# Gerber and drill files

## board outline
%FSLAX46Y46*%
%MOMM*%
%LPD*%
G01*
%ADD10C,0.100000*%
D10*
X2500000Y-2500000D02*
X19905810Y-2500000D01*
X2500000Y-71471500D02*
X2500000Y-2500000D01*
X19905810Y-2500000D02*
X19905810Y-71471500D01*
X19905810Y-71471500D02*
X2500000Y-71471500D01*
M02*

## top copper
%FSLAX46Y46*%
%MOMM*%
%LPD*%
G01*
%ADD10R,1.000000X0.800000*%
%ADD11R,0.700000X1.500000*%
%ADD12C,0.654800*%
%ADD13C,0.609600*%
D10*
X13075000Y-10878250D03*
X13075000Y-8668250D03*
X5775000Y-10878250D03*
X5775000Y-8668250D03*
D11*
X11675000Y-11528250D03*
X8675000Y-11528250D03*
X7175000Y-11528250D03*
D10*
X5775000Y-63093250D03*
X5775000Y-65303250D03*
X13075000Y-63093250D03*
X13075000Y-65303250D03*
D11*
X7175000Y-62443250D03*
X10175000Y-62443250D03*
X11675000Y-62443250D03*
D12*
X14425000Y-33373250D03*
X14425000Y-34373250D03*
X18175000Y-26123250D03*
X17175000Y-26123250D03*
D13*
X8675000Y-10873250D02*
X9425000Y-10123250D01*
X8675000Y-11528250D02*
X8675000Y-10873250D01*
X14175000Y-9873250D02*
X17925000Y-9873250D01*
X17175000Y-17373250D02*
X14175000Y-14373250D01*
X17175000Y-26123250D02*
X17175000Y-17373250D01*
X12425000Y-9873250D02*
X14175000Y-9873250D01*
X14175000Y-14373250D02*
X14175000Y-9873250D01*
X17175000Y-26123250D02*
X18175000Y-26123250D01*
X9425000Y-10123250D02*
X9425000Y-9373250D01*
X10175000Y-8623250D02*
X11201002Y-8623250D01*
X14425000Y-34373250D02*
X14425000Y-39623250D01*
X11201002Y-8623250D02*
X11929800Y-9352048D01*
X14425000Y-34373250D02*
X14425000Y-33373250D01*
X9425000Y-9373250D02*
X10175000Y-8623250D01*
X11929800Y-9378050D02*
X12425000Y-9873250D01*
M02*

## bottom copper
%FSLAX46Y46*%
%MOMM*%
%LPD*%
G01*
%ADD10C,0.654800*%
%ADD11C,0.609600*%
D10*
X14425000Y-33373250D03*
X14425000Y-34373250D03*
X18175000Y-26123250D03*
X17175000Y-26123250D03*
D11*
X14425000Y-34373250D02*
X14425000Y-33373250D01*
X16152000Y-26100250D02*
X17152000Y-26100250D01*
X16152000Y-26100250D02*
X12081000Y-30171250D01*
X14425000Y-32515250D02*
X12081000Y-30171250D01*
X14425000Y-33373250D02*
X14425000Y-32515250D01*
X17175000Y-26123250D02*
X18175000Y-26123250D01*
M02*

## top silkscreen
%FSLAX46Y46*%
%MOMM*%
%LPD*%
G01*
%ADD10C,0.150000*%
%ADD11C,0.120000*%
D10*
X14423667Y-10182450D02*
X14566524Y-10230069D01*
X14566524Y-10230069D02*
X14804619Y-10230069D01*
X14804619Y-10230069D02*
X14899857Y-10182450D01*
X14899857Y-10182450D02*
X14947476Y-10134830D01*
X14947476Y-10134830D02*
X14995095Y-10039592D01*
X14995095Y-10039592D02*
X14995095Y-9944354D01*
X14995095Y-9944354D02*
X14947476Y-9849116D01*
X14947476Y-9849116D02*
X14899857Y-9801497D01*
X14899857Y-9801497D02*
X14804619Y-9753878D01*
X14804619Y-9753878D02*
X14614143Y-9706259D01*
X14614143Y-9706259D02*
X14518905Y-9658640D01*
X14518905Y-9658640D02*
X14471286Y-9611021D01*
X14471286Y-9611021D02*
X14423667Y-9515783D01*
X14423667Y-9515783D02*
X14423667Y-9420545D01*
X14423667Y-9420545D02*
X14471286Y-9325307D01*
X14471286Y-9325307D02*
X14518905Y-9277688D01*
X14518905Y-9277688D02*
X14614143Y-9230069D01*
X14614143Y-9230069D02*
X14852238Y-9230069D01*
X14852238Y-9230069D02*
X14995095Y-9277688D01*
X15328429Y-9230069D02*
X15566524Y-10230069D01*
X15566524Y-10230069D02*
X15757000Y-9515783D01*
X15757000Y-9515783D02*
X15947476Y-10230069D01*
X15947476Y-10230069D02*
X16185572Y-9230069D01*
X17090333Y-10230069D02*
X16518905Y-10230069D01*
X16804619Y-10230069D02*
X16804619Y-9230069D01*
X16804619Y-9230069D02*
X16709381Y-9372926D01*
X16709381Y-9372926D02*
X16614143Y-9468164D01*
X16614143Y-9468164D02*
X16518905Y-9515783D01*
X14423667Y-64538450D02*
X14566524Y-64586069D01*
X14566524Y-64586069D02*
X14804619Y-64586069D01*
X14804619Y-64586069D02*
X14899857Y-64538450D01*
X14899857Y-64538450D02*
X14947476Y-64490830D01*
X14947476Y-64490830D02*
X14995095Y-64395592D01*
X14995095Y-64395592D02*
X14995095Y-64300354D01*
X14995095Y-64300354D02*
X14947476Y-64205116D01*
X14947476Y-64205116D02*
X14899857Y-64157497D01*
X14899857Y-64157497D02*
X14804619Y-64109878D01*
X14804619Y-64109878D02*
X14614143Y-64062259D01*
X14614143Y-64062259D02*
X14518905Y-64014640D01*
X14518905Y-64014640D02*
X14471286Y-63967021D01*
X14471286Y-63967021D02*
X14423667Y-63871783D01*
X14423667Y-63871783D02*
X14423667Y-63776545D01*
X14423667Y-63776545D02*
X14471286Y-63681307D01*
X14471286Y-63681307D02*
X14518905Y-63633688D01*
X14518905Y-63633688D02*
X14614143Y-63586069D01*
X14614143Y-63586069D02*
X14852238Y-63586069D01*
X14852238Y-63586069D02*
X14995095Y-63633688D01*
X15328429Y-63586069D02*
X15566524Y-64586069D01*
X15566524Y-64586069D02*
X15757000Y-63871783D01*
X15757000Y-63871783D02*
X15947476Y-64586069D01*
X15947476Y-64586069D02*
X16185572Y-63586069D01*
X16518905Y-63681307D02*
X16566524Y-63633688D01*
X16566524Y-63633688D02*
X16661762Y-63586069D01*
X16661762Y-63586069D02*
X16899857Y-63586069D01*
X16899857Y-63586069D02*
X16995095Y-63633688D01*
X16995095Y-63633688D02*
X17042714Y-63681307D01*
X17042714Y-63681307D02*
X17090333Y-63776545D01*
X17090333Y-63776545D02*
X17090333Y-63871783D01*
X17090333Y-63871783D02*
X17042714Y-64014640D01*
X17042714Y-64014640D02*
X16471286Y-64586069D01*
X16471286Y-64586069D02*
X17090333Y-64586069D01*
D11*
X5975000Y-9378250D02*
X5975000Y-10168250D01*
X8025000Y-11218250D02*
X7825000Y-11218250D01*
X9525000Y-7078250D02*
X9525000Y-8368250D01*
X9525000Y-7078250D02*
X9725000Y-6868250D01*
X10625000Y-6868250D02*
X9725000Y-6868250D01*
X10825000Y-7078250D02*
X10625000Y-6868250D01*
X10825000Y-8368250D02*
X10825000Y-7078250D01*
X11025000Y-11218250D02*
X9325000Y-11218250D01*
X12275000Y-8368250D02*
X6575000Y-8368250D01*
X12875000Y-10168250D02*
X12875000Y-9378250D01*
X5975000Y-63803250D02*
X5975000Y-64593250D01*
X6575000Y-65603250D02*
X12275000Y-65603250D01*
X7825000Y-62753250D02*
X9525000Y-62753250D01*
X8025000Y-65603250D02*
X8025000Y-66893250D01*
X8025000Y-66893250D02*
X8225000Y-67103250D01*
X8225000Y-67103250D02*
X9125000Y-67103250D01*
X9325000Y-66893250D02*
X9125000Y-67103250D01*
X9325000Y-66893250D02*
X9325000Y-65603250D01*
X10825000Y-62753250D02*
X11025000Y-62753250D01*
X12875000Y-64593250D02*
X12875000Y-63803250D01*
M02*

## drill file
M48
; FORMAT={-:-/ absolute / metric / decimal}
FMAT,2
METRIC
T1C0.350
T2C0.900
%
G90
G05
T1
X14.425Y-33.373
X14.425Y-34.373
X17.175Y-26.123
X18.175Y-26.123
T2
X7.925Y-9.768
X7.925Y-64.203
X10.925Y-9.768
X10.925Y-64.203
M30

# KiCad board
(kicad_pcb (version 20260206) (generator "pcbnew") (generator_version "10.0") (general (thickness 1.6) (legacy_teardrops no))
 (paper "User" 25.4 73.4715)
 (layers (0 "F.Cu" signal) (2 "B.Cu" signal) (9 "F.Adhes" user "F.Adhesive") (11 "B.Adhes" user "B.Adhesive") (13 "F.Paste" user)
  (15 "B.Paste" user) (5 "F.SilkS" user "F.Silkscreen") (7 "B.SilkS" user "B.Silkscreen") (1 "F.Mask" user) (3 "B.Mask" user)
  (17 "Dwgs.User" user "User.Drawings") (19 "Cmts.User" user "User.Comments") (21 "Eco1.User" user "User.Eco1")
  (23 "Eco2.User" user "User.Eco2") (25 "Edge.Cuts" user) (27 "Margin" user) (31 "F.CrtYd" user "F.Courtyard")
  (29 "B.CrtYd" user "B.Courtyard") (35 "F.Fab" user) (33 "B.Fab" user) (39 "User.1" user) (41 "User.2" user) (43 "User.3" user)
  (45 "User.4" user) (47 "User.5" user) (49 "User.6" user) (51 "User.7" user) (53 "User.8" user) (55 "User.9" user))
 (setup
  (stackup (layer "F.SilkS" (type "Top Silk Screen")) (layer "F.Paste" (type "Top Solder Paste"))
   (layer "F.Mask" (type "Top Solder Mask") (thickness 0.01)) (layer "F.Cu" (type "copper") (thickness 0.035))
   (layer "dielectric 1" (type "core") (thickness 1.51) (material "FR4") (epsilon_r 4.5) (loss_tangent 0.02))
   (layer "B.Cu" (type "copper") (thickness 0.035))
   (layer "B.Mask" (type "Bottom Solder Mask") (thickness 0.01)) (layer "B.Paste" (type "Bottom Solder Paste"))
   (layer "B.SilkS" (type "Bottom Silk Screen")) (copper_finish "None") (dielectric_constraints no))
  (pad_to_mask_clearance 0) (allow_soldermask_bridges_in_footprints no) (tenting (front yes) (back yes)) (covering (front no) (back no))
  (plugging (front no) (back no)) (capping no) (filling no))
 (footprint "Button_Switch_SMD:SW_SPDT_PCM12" (layer "F.Cu") (at 9.425 10.09825 180)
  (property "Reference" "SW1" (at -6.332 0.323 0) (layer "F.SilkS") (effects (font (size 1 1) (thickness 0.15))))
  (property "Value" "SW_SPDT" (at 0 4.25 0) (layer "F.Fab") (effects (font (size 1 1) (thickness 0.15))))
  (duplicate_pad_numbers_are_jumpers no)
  (fp_line (start 3.45 0.72) (end 3.45 -0.07) (stroke (width 0.12) (type solid)) (layer "F.SilkS"))
  (fp_line (start 1.4 -1.12) (end 1.6 -1.12) (stroke (width 0.12) (type solid)) (layer "F.SilkS"))
  (fp_line (start -0.1 3.02) (end -0.1 1.73) (stroke (width 0.12) (type solid)) (layer "F.SilkS"))
  (fp_line (start -0.1 3.02) (end -0.3 3.23) (stroke (width 0.12) (type solid)) (layer "F.SilkS"))
  (fp_line (start -1.2 3.23) (end -0.3 3.23) (stroke (width 0.12) (type solid)) (layer "F.SilkS"))
  (fp_line (start -1.4 3.02) (end -1.2 3.23) (stroke (width 0.12) (type solid)) (layer "F.SilkS"))
  (fp_line (start -1.4 1.73) (end -1.4 3.02) (stroke (width 0.12) (type solid)) (layer "F.SilkS"))
  (fp_line (start -1.6 -1.12) (end 0.1 -1.12) (stroke (width 0.12) (type solid)) (layer "F.SilkS"))
  (fp_line (start -2.85 1.73) (end 2.85 1.73) (stroke (width 0.12) (type solid)) (layer "F.SilkS"))
  (fp_line (start -3.45 -0.07) (end -3.45 0.72) (stroke (width 0.12) (type solid)) (layer "F.SilkS"))
  (pad "" smd rect (at -3.65 -0.78 180) (size 1 0.8) (layers "F.Cu" "F.Mask" "F.Paste"))
  (pad "" smd rect (at -3.65 1.43 180) (size 1 0.8) (layers "F.Cu" "F.Mask" "F.Paste"))
  (pad "" np_thru_hole circle (at -1.5 0.33 180) (size 0.9 0.9) (drill 0.9) (layers "*.Cu" "*.Mask"))
  (pad "" np_thru_hole circle (at 1.5 0.33 180) (size 0.9 0.9) (drill 0.9) (layers "*.Cu" "*.Mask"))
  (pad "" smd rect (at 3.65 -0.78 180) (size 1 0.8) (layers "F.Cu" "F.Mask" "F.Paste"))
  (pad "" smd rect (at 3.65 1.43 180) (size 1 0.8) (layers "F.Cu" "F.Mask" "F.Paste"))
  (pad "1" smd rect (at -2.25 -1.43 180) (size 0.7 1.5) (layers "F.Cu" "F.Mask" "F.Paste") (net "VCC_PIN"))
  (pad "2" smd rect (at 0.75 -1.43 180) (size 0.7 1.5) (layers "F.Cu" "F.Mask" "F.Paste") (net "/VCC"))
  (pad "3" smd rect (at 2.25 -1.43 180) (size 0.7 1.5) (layers "F.Cu" "F.Mask" "F.Paste") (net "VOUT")))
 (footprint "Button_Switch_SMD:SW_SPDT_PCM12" (layer "F.Cu") (at 9.425 63.87325)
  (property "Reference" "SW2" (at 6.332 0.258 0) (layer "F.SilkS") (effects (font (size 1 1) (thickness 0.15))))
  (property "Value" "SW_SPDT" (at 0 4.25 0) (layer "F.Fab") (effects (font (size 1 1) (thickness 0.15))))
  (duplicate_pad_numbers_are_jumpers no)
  (fp_line (start -3.45 -0.07) (end -3.45 0.72) (stroke (width 0.12) (type solid)) (layer "F.SilkS"))
  (fp_line (start -2.85 1.73) (end 2.85 1.73) (stroke (width 0.12) (type solid)) (layer "F.SilkS"))
  (fp_line (start -1.6 -1.12) (end 0.1 -1.12) (stroke (width 0.12) (type solid)) (layer "F.SilkS"))
  (fp_line (start -1.4 1.73) (end -1.4 3.02) (stroke (width 0.12) (type solid)) (layer "F.SilkS"))
  (fp_line (start -1.4 3.02) (end -1.2 3.23) (stroke (width 0.12) (type solid)) (layer "F.SilkS"))
  (fp_line (start -1.2 3.23) (end -0.3 3.23) (stroke (width 0.12) (type solid)) (layer "F.SilkS"))
  (fp_line (start -0.1 3.02) (end -0.3 3.23) (stroke (width 0.12) (type solid)) (layer "F.SilkS"))
  (fp_line (start -0.1 3.02) (end -0.1 1.73) (stroke (width 0.12) (type solid)) (layer "F.SilkS"))
  (fp_line (start 1.4 -1.12) (end 1.6 -1.12) (stroke (width 0.12) (type solid)) (layer "F.SilkS"))
  (fp_line (start 3.45 0.72) (end 3.45 -0.07) (stroke (width 0.12) (type solid)) (layer "F.SilkS"))
  (pad "" smd rect (at -3.65 -0.78) (size 1 0.8) (layers "F.Cu" "F.Mask" "F.Paste"))
  (pad "" smd rect (at -3.65 1.43) (size 1 0.8) (layers "F.Cu" "F.Mask" "F.Paste"))
  (pad "" np_thru_hole circle (at -1.5 0.33) (size 0.9 0.9) (drill 0.9) (layers "*.Cu" "*.Mask"))
  (pad "" np_thru_hole circle (at 1.5 0.33) (size 0.9 0.9) (drill 0.9) (layers "*.Cu" "*.Mask"))
  (pad "" smd rect (at 3.65 -0.78) (size 1 0.8) (layers "F.Cu" "F.Mask" "F.Paste"))
  (pad "" smd rect (at 3.65 1.43) (size 1 0.8) (layers "F.Cu" "F.Mask" "F.Paste"))
  (pad "1" smd rect (at -2.25 -1.43) (size 0.7 1.5) (layers "F.Cu" "F.Mask" "F.Paste") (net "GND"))
  (pad "2" smd rect (at 0.75 -1.43) (size 0.7 1.5) (layers "F.Cu" "F.Mask" "F.Paste") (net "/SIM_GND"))
  (pad "3" smd rect (at 2.25 -1.43) (size 0.7 1.5) (layers "F.Cu" "F.Mask" "F.Paste") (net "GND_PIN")))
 (gr_line (start 2.5 2.5) (end 19.90581 2.5) (stroke (width 0.1) (type default)) (layer "Edge.Cuts"))
 (gr_line (start 2.5 71.4715) (end 2.5 2.5) (stroke (width 0.1) (type default)) (layer "Edge.Cuts"))
 (gr_line (start 19.90581 2.5) (end 19.90581 71.4715) (stroke (width 0.1) (type default)) (layer "Edge.Cuts"))
 (gr_line (start 19.90581 71.4715) (end 2.5 71.4715) (stroke (width 0.1) (type default)) (layer "Edge.Cuts"))
 (segment (start 8.675 10.87325) (end 9.425 10.12325) (width 0.6096) (layer "F.Cu") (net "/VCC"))
 (segment (start 8.675 11.52825) (end 8.675 10.87325) (width 0.6096) (layer "F.Cu") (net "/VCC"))
 (segment (start 14.175 9.87325) (end 17.925 9.87325) (width 0.6096) (layer "F.Cu") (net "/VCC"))
 (segment (start 17.175 17.37325) (end 14.175 14.37325) (width 0.6096) (layer "F.Cu") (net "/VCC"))
 (segment (start 17.175 26.12325) (end 17.175 17.37325) (width 0.6096) (layer "F.Cu") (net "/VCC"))
 (segment (start 12.425 9.87325) (end 14.175 9.87325) (width 0.6096) (layer "F.Cu") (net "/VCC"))
 (segment (start 14.175 14.37325) (end 14.175 9.87325) (width 0.6096) (layer "F.Cu") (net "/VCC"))
 (segment (start 17.175 26.12325) (end 18.175 26.12325) (width 0.6096) (layer "F.Cu") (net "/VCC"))
 (segment (start 9.425 10.12325) (end 9.425 9.37325) (width 0.6096) (layer "F.Cu") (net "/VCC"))
 (segment (start 10.175 8.62325) (end 11.201002 8.62325) (width 0.6096) (layer "F.Cu") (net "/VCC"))
 (segment (start 14.425 34.37325) (end 14.425 39.62325) (width 0.6096) (layer "F.Cu") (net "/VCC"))
 (segment (start 11.201002 8.62325) (end 11.9298 9.352048) (width 0.6096) (layer "F.Cu") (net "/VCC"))
 (segment (start 14.425 34.37325) (end 14.425 33.37325) (width 0.6096) (layer "F.Cu") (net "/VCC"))
 (segment (start 9.425 9.37325) (end 10.175 8.62325) (width 0.6096) (layer "F.Cu") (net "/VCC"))
 (segment (start 11.9298 9.37805) (end 12.425 9.87325) (width 0.6096) (layer "F.Cu") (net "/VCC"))
 (via (at 14.425 33.37325) (size 0.6548) (drill 0.35) (layers "F.Cu" "B.Cu") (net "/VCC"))
 (via (at 14.425 34.37325) (size 0.6548) (drill 0.35) (layers "F.Cu" "B.Cu") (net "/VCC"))
 (via (at 18.175 26.12325) (size 0.6548) (drill 0.35) (layers "F.Cu" "B.Cu") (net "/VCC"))
 (via (at 17.175 26.12325) (size 0.6548) (drill 0.35) (layers "F.Cu" "B.Cu") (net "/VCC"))
 (segment (start 14.425 34.37325) (end 14.425 33.37325) (width 0.6096) (layer "B.Cu") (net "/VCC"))
 (segment (start 16.152 26.10025) (end 17.152 26.10025) (width 0.6096) (layer "B.Cu") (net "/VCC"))
 (segment (start 16.152 26.10025) (end 12.081 30.17125) (width 0.6096) (layer "B.Cu") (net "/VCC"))
 (segment (start 14.425 32.51525) (end 12.081 30.17125) (width 0.6096) (layer "B.Cu") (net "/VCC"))
 (segment (start 14.425 33.37325) (end 14.425 32.51525) (width 0.6096) (layer "B.Cu") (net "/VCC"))
 (segment (start 17.175 26.12325) (end 18.175 26.12325) (width 0.6096) (layer "B.Cu") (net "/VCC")))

